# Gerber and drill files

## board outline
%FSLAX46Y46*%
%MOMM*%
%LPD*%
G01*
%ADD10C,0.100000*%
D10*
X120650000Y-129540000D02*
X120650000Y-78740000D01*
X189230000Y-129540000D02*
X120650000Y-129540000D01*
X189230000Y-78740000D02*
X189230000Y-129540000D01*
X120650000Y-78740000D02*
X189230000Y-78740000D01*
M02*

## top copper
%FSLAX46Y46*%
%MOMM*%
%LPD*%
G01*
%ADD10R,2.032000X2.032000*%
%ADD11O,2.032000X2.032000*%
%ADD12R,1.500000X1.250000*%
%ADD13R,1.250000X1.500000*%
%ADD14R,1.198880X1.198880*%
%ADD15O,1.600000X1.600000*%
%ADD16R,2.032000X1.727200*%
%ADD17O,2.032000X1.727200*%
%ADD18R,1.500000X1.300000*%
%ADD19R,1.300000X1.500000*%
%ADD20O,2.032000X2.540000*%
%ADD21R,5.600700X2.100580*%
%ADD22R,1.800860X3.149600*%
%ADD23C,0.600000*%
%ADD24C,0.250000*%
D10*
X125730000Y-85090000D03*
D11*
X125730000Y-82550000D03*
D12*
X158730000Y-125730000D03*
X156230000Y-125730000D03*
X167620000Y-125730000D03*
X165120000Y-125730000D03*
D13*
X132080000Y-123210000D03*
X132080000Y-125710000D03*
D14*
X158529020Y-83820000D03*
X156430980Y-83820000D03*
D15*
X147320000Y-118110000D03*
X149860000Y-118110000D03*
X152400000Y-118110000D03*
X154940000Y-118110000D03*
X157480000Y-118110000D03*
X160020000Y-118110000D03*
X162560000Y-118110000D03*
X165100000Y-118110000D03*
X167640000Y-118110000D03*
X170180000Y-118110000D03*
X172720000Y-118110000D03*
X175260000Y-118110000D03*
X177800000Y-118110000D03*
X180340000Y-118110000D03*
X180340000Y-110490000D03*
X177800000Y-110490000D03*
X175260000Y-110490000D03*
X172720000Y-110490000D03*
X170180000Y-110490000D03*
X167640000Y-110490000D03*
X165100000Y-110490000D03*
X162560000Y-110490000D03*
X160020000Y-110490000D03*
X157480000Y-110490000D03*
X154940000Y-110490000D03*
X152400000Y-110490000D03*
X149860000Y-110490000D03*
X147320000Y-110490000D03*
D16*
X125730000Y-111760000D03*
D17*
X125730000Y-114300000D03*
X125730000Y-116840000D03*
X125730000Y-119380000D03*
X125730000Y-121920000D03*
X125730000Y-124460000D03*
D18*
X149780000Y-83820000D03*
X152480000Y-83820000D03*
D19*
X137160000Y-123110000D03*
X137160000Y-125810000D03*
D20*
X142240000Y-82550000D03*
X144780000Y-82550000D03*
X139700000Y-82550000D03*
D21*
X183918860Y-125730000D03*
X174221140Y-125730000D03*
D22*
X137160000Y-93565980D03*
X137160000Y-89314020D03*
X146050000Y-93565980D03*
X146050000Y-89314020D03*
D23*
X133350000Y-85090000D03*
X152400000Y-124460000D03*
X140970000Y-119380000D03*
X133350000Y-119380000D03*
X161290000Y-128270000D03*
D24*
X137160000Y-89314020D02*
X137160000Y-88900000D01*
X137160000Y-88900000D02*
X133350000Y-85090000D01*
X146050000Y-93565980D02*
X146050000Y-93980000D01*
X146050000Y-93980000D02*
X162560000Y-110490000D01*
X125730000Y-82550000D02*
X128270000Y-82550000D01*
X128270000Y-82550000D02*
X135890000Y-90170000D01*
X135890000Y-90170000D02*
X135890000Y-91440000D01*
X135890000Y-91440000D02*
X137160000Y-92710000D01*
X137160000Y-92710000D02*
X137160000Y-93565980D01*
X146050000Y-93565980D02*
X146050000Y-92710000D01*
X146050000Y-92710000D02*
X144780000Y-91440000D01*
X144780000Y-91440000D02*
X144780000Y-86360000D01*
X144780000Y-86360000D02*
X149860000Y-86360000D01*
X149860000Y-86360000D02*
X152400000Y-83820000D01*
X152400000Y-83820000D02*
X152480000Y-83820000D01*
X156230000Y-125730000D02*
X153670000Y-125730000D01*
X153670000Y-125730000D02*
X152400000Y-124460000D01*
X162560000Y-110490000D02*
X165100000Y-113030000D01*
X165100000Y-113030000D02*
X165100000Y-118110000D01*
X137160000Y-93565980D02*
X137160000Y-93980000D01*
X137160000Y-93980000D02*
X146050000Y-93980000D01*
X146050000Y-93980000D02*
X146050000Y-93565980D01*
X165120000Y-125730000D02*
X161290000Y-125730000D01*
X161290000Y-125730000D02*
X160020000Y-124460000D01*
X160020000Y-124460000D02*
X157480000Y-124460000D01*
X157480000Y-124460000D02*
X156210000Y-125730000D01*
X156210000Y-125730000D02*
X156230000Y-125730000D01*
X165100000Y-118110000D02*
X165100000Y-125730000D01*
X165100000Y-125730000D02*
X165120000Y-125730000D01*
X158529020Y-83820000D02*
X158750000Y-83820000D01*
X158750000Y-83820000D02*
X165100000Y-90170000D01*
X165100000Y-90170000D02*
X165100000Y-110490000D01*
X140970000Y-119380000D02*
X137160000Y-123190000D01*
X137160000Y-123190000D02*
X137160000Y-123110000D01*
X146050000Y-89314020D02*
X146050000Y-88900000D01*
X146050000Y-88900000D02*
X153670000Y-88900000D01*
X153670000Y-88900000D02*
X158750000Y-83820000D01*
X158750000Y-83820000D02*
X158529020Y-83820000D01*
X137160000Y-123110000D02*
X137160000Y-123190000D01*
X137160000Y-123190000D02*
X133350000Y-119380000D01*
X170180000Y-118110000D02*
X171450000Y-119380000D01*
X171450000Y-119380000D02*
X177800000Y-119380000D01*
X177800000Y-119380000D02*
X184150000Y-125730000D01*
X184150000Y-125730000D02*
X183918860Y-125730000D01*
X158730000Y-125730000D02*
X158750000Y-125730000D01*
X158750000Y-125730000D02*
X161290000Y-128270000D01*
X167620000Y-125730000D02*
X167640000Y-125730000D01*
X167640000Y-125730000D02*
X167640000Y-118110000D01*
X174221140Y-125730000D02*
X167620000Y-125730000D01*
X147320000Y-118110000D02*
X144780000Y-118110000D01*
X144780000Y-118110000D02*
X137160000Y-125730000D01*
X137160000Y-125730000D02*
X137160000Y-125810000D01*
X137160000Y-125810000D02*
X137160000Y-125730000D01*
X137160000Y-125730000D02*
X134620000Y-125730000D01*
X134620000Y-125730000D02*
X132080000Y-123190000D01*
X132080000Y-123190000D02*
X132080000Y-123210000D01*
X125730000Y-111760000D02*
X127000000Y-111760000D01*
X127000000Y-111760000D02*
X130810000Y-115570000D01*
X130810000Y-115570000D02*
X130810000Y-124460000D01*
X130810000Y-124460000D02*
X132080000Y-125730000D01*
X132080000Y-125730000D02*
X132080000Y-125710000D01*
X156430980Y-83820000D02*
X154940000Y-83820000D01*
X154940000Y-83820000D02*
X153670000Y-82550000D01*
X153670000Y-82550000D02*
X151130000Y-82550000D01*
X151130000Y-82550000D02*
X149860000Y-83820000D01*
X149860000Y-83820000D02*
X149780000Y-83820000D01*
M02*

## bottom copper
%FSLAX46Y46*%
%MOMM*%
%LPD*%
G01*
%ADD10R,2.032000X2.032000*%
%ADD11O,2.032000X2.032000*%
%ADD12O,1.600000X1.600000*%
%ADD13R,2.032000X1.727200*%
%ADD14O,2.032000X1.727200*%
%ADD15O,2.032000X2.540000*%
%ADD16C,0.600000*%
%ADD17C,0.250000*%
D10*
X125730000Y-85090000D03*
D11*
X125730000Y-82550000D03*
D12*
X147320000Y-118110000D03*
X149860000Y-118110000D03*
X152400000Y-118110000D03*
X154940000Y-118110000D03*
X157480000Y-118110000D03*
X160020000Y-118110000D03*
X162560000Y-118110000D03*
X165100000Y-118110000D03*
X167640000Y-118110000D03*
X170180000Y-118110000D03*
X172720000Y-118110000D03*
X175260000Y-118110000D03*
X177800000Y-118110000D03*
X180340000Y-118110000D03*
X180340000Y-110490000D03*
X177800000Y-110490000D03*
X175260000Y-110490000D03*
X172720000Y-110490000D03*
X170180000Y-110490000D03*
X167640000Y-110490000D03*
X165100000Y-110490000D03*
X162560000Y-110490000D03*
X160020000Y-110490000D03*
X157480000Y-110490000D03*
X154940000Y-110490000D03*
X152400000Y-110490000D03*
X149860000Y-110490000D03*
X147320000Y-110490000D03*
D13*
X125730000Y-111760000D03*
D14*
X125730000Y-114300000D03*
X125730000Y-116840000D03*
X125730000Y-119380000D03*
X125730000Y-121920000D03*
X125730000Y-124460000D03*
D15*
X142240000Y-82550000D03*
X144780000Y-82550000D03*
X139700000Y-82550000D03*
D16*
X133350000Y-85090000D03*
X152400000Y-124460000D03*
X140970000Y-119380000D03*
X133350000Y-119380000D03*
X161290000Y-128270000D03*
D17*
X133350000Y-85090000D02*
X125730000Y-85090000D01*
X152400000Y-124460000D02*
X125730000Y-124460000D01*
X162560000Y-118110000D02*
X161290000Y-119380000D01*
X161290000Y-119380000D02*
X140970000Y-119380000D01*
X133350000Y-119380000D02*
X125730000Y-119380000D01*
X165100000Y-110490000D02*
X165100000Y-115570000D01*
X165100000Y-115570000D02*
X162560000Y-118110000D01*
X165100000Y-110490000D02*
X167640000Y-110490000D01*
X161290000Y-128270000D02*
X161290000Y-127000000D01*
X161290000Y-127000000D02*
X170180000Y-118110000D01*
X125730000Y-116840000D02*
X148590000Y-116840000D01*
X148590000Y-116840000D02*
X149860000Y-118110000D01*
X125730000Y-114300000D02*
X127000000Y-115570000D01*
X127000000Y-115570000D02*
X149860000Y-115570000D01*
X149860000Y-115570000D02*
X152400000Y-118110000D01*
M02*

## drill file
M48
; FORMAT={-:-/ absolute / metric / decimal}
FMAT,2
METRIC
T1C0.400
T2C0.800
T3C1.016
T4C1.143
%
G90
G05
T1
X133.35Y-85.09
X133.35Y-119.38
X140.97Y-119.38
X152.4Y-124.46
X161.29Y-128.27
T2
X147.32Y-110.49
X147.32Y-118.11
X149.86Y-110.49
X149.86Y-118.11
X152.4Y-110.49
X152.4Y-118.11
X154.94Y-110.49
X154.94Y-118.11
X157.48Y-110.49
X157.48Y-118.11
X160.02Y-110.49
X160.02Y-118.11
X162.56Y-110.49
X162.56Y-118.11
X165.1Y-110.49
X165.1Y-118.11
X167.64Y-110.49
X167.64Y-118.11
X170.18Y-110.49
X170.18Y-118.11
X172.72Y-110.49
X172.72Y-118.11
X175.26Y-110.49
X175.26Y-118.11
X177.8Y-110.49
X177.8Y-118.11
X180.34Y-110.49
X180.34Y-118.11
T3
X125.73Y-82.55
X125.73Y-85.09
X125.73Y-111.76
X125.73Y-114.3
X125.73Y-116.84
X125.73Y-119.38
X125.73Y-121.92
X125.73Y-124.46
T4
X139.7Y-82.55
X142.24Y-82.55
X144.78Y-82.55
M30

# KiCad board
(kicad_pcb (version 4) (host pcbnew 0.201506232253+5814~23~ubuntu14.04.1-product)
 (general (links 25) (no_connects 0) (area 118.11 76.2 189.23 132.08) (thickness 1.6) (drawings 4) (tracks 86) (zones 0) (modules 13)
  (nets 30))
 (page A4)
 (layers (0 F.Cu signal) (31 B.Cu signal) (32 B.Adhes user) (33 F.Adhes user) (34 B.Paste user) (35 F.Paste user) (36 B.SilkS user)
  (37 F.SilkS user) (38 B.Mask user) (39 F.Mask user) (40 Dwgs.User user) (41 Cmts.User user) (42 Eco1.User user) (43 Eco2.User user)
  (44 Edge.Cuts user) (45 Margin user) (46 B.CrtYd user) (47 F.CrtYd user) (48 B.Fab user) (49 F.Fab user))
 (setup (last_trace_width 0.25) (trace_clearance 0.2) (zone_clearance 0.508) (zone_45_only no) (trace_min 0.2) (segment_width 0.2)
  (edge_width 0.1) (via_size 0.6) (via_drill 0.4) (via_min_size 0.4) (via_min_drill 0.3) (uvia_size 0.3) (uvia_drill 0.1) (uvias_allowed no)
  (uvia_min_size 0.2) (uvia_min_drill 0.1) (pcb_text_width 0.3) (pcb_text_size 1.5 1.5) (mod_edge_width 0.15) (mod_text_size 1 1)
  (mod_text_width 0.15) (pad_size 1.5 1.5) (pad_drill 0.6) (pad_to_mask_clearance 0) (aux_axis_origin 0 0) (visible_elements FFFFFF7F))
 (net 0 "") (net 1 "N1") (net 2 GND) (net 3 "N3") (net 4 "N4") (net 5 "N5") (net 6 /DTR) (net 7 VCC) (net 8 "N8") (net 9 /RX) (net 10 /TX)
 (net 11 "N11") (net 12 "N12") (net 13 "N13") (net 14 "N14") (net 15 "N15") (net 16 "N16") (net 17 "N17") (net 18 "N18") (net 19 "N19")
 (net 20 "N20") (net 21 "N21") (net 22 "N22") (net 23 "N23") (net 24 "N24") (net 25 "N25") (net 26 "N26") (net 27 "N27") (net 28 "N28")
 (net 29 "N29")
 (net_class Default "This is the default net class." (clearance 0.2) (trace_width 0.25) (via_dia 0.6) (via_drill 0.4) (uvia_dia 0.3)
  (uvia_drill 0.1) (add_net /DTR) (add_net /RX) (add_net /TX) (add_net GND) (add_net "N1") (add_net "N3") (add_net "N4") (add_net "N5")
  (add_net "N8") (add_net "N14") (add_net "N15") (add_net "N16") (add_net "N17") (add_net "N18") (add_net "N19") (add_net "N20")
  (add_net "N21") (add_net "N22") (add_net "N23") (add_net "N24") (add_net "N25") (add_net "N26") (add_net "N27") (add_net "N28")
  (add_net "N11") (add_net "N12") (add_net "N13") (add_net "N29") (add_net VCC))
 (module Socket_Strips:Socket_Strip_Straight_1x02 (layer F.Cu) (at 125.73 85.09 90)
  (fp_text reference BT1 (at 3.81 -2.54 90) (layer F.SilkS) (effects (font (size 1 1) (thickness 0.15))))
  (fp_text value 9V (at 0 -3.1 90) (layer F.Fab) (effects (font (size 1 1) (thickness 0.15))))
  (pad 1 thru_hole rect (at 0 0 90) (size 2.032 2.032) (drill 1.016) (layers *.Cu *.Mask F.SilkS) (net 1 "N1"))
  (pad 2 thru_hole oval (at 2.54 0 90) (size 2.032 2.032) (drill 1.016) (layers *.Cu *.Mask F.SilkS) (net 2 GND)))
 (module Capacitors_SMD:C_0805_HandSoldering (layer F.Cu) (at 157.48 125.73 180)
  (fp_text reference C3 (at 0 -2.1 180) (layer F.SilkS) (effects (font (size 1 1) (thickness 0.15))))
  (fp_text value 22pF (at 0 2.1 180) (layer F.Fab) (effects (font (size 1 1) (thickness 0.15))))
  (pad 1 smd rect (at -1.25 0 180) (size 1.5 1.25) (layers F.Cu F.Paste F.Mask) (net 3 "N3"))
  (pad 2 smd rect (at 1.25 0 180) (size 1.5 1.25) (layers F.Cu F.Paste F.Mask) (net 2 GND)))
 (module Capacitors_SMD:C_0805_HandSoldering (layer F.Cu) (at 166.37 125.73 180)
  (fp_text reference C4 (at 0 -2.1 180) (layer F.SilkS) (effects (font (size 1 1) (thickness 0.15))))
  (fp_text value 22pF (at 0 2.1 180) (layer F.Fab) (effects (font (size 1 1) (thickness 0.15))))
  (pad 1 smd rect (at -1.25 0 180) (size 1.5 1.25) (layers F.Cu F.Paste F.Mask) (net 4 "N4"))
  (pad 2 smd rect (at 1.25 0 180) (size 1.5 1.25) (layers F.Cu F.Paste F.Mask) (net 2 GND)))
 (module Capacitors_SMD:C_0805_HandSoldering (layer F.Cu) (at 132.08 124.46 270)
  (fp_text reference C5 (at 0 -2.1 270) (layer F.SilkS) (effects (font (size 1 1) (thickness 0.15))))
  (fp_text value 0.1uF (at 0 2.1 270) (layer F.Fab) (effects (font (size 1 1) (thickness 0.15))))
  (pad 1 smd rect (at -1.25 0 270) (size 1.5 1.25) (layers F.Cu F.Paste F.Mask) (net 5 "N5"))
  (pad 2 smd rect (at 1.25 0 270) (size 1.5 1.25) (layers F.Cu F.Paste F.Mask) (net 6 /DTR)))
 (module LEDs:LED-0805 (layer F.Cu) (at 157.48 83.82)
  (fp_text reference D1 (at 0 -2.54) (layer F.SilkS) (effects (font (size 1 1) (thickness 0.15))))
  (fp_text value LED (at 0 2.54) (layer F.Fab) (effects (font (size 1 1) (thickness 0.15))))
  (pad 2 smd rect (at 1.04902 0 180) (size 1.19888 1.19888) (layers F.Cu F.Paste F.Mask) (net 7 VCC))
  (pad 1 smd rect (at -1.04902 0 180) (size 1.19888 1.19888) (layers F.Cu F.Paste F.Mask) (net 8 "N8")))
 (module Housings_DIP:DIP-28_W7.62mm (layer F.Cu) (at 147.32 118.11 90)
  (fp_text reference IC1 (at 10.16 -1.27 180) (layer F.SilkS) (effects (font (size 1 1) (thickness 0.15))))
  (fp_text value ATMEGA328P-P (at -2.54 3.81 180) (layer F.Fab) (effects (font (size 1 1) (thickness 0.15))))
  (pad 1 thru_hole oval (at 0 0 90) (size 1.6 1.6) (drill 0.8) (layers *.Cu *.Mask F.SilkS) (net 5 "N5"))
  (pad 2 thru_hole oval (at 0 2.54 90) (size 1.6 1.6) (drill 0.8) (layers *.Cu *.Mask F.SilkS) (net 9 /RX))
  (pad 3 thru_hole oval (at 0 5.08 90) (size 1.6 1.6) (drill 0.8) (layers *.Cu *.Mask F.SilkS) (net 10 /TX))
  (pad 4 thru_hole oval (at 0 7.62 90) (size 1.6 1.6) (drill 0.8) (layers *.Cu *.Mask F.SilkS) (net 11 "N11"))
  (pad 5 thru_hole oval (at 0 10.16 90) (size 1.6 1.6) (drill 0.8) (layers *.Cu *.Mask F.SilkS) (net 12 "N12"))
  (pad 6 thru_hole oval (at 0 12.7 90) (size 1.6 1.6) (drill 0.8) (layers *.Cu *.Mask F.SilkS) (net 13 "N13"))
  (pad 7 thru_hole oval (at 0 15.24 90) (size 1.6 1.6) (drill 0.8) (layers *.Cu *.Mask F.SilkS) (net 7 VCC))
  (pad 8 thru_hole oval (at 0 17.78 90) (size 1.6 1.6) (drill 0.8) (layers *.Cu *.Mask F.SilkS) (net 2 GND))
  (pad 9 thru_hole oval (at 0 20.32 90) (size 1.6 1.6) (drill 0.8) (layers *.Cu *.Mask F.SilkS) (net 4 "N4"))
  (pad 10 thru_hole oval (at 0 22.86 90) (size 1.6 1.6) (drill 0.8) (layers *.Cu *.Mask F.SilkS) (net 3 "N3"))
  (pad 11 thru_hole oval (at 0 25.4 90) (size 1.6 1.6) (drill 0.8) (layers *.Cu *.Mask F.SilkS) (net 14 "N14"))
  (pad 12 thru_hole oval (at 0 27.94 90) (size 1.6 1.6) (drill 0.8) (layers *.Cu *.Mask F.SilkS) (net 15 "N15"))
  (pad 13 thru_hole oval (at 0 30.48 90) (size 1.6 1.6) (drill 0.8) (layers *.Cu *.Mask F.SilkS) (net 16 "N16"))
  (pad 14 thru_hole oval (at 0 33.02 90) (size 1.6 1.6) (drill 0.8) (layers *.Cu *.Mask F.SilkS) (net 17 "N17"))
  (pad 15 thru_hole oval (at 7.62 33.02 90) (size 1.6 1.6) (drill 0.8) (layers *.Cu *.Mask F.SilkS) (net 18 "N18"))
  (pad 16 thru_hole oval (at 7.62 30.48 90) (size 1.6 1.6) (drill 0.8) (layers *.Cu *.Mask F.SilkS) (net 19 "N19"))
  (pad 17 thru_hole oval (at 7.62 27.94 90) (size 1.6 1.6) (drill 0.8) (layers *.Cu *.Mask F.SilkS) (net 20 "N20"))
  (pad 18 thru_hole oval (at 7.62 25.4 90) (size 1.6 1.6) (drill 0.8) (layers *.Cu *.Mask F.SilkS) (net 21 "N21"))
  (pad 19 thru_hole oval (at 7.62 22.86 90) (size 1.6 1.6) (drill 0.8) (layers *.Cu *.Mask F.SilkS) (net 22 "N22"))
  (pad 20 thru_hole oval (at 7.62 20.32 90) (size 1.6 1.6) (drill 0.8) (layers *.Cu *.Mask F.SilkS) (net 7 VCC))
  (pad 21 thru_hole oval (at 7.62 17.78 90) (size 1.6 1.6) (drill 0.8) (layers *.Cu *.Mask F.SilkS) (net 7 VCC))
  (pad 22 thru_hole oval (at 7.62 15.24 90) (size 1.6 1.6) (drill 0.8) (layers *.Cu *.Mask F.SilkS) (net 2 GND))
  (pad 23 thru_hole oval (at 7.62 12.7 90) (size 1.6 1.6) (drill 0.8) (layers *.Cu *.Mask F.SilkS) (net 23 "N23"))
  (pad 24 thru_hole oval (at 7.62 10.16 90) (size 1.6 1.6) (drill 0.8) (layers *.Cu *.Mask F.SilkS) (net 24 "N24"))
  (pad 25 thru_hole oval (at 7.62 7.62 90) (size 1.6 1.6) (drill 0.8) (layers *.Cu *.Mask F.SilkS) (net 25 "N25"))
  (pad 26 thru_hole oval (at 7.62 5.08 90) (size 1.6 1.6) (drill 0.8) (layers *.Cu *.Mask F.SilkS) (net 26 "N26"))
  (pad 27 thru_hole oval (at 7.62 2.54 90) (size 1.6 1.6) (drill 0.8) (layers *.Cu *.Mask F.SilkS) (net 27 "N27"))
  (pad 28 thru_hole oval (at 7.62 0 90) (size 1.6 1.6) (drill 0.8) (layers *.Cu *.Mask F.SilkS) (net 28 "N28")))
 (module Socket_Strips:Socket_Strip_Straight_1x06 (layer F.Cu) (at 125.73 111.76 270)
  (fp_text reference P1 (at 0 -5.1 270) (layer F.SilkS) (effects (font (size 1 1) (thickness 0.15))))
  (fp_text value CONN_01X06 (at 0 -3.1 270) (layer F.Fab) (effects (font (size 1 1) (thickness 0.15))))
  (pad 1 thru_hole rect (at 0 0 270) (size 1.7272 2.032) (drill 1.016) (layers *.Cu *.Mask F.SilkS) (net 6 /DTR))
  (pad 2 thru_hole oval (at 2.54 0 270) (size 1.7272 2.032) (drill 1.016) (layers *.Cu *.Mask F.SilkS) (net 10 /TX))
  (pad 3 thru_hole oval (at 5.08 0 270) (size 1.7272 2.032) (drill 1.016) (layers *.Cu *.Mask F.SilkS) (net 9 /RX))
  (pad 4 thru_hole oval (at 7.62 0 270) (size 1.7272 2.032) (drill 1.016) (layers *.Cu *.Mask F.SilkS) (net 7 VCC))
  (pad 5 thru_hole oval (at 10.16 0 270) (size 1.7272 2.032) (drill 1.016) (layers *.Cu *.Mask F.SilkS) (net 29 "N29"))
  (pad 6 thru_hole oval (at 12.7 0 270) (size 1.7272 2.032) (drill 1.016) (layers *.Cu *.Mask F.SilkS) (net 2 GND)))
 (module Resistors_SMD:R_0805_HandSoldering (layer F.Cu) (at 151.13 83.82)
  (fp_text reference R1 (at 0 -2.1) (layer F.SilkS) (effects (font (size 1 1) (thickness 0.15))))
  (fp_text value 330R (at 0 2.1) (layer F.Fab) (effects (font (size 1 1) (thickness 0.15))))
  (pad 1 smd rect (at -1.35 0) (size 1.5 1.3) (layers F.Cu F.Paste F.Mask) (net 8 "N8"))
  (pad 2 smd rect (at 1.35 0) (size 1.5 1.3) (layers F.Cu F.Paste F.Mask) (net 2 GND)))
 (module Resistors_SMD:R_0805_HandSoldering (layer F.Cu) (at 137.16 124.46 270)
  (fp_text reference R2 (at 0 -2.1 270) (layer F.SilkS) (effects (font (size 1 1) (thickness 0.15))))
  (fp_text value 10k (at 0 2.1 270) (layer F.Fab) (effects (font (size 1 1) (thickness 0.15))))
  (pad 1 smd rect (at -1.35 0 270) (size 1.5 1.3) (layers F.Cu F.Paste F.Mask) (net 7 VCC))
  (pad 2 smd rect (at 1.35 0 270) (size 1.5 1.3) (layers F.Cu F.Paste F.Mask) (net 5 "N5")))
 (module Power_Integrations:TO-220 (layer F.Cu) (at 142.24 82.55)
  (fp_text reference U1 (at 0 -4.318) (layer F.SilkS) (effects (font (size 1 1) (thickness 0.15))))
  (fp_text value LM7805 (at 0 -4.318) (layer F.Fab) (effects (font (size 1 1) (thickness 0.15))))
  (pad 2 thru_hole oval (at 0 0) (size 2.032 2.54) (drill 1.143) (layers *.Cu *.Mask F.SilkS))
  (pad 3 thru_hole oval (at 2.54 0) (size 2.032 2.54) (drill 1.143) (layers *.Cu *.Mask F.SilkS))
  (pad 1 thru_hole oval (at -2.54 0) (size 2.032 2.54) (drill 1.143) (layers *.Cu *.Mask F.SilkS)))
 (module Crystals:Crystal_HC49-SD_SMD (layer F.Cu) (at 179.07 125.73 180)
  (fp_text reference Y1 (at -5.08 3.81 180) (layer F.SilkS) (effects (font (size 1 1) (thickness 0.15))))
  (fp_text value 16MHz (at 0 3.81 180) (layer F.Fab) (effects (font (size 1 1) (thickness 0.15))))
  (pad 1 smd rect (at -4.84886 0 180) (size 5.6007 2.10058) (layers F.Cu F.Paste F.Mask) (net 3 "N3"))
  (pad 2 smd rect (at 4.84886 0 180) (size 5.6007 2.10058) (layers F.Cu F.Paste F.Mask) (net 4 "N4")))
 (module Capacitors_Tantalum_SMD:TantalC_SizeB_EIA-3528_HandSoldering (layer F.Cu) (at 137.16 91.44 270)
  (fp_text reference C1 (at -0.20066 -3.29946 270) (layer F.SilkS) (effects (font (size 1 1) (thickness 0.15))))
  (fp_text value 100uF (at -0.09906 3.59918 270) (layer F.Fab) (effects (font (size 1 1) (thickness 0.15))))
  (pad 2 smd rect (at 2.12598 0 270) (size 3.1496 1.80086) (layers F.Cu F.Paste F.Mask) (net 2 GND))
  (pad 1 smd rect (at -2.12598 0 270) (size 3.1496 1.80086) (layers F.Cu F.Paste F.Mask) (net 1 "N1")))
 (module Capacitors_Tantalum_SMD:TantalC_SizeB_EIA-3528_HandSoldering (layer F.Cu) (at 146.05 91.44 270)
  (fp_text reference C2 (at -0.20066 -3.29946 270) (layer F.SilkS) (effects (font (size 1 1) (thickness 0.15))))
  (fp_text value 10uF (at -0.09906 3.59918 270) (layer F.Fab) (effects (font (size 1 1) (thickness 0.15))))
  (pad 2 smd rect (at 2.12598 0 270) (size 3.1496 1.80086) (layers F.Cu F.Paste F.Mask) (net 2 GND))
  (pad 1 smd rect (at -2.12598 0 270) (size 3.1496 1.80086) (layers F.Cu F.Paste F.Mask) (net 7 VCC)))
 (gr_line (start 120.65 129.54) (end 120.65 78.74) (angle 90) (layer Edge.Cuts) (width 0.1))
 (gr_line (start 189.23 129.54) (end 120.65 129.54) (angle 90) (layer Edge.Cuts) (width 0.1))
 (gr_line (start 189.23 78.74) (end 189.23 129.54) (angle 90) (layer Edge.Cuts) (width 0.1))
 (gr_line (start 120.65 78.74) (end 189.23 78.74) (angle 90) (layer Edge.Cuts) (width 0.1))
 (segment (start 137.16 89.31402) (end 137.16 88.9) (width 0.25) (layer F.Cu) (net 1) (status 80000))
 (segment (start 137.16 88.9) (end 133.35 85.09) (width 0.25) (layer F.Cu) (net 1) (status 80000))
 (segment (start 133.35 85.09) (end 125.73 85.09) (width 0.25) (layer B.Cu) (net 1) (status 80000))
 (segment (start 146.05 93.56598) (end 146.05 93.98) (width 0.25) (layer F.Cu) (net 2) (status 80000))
 (segment (start 146.05 93.98) (end 162.56 110.49) (width 0.25) (layer F.Cu) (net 2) (status 80000))
 (segment (start 125.73 82.55) (end 128.27 82.55) (width 0.25) (layer F.Cu) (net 2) (status 80000))
 (segment (start 128.27 82.55) (end 135.89 90.17) (width 0.25) (layer F.Cu) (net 2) (status 80000))
 (segment (start 135.89 90.17) (end 135.89 91.44) (width 0.25) (layer F.Cu) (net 2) (status 80000))
 (segment (start 135.89 91.44) (end 137.16 92.71) (width 0.25) (layer F.Cu) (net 2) (status 80000))
 (segment (start 137.16 92.71) (end 137.16 93.56598) (width 0.25) (layer F.Cu) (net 2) (status 80000))
 (segment (start 146.05 93.56598) (end 146.05 92.71) (width 0.25) (layer F.Cu) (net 2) (status 80000))
 (segment (start 146.05 92.71) (end 144.78 91.44) (width 0.25) (layer F.Cu) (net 2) (status 80000))
 (segment (start 144.78 91.44) (end 144.78 86.36) (width 0.25) (layer F.Cu) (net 2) (status 80000))
 (segment (start 144.78 86.36) (end 149.86 86.36) (width 0.25) (layer F.Cu) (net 2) (status 80000))
 (segment (start 149.86 86.36) (end 152.4 83.82) (width 0.25) (layer F.Cu) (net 2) (status 80000))
 (segment (start 152.4 83.82) (end 152.48 83.82) (width 0.25) (layer F.Cu) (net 2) (status 80000))
 (segment (start 156.23 125.73) (end 153.67 125.73) (width 0.25) (layer F.Cu) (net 2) (status 80000))
 (segment (start 153.67 125.73) (end 152.4 124.46) (width 0.25) (layer F.Cu) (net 2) (status 80000))
 (segment (start 152.4 124.46) (end 125.73 124.46) (width 0.25) (layer B.Cu) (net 2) (status 80000))
 (segment (start 162.56 110.49) (end 165.1 113.03) (width 0.25) (layer F.Cu) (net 2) (status 80000))
 (segment (start 165.1 113.03) (end 165.1 118.11) (width 0.25) (layer F.Cu) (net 2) (status 80000))
 (segment (start 137.16 93.56598) (end 137.16 93.98) (width 0.25) (layer F.Cu) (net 2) (status 80000))
 (segment (start 137.16 93.98) (end 146.05 93.98) (width 0.25) (layer F.Cu) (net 2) (status 80000))
 (segment (start 146.05 93.98) (end 146.05 93.56598) (width 0.25) (layer F.Cu) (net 2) (status 80000))
 (segment (start 165.12 125.73) (end 161.29 125.73) (width 0.25) (layer F.Cu) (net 2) (status 80000))
 (segment (start 161.29 125.73) (end 160.02 124.46) (width 0.25) (layer F.Cu) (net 2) (status 80000))
 (segment (start 160.02 124.46) (end 157.48 124.46) (width 0.25) (layer F.Cu) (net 2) (status 80000))
 (segment (start 157.48 124.46) (end 156.21 125.73) (width 0.25) (layer F.Cu) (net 2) (status 80000))
 (segment (start 156.21 125.73) (end 156.23 125.73) (width 0.25) (layer F.Cu) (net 2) (status 80000))
 (segment (start 165.1 118.11) (end 165.1 125.73) (width 0.25) (layer F.Cu) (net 2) (status 80000))
 (segment (start 165.1 125.73) (end 165.12 125.73) (width 0.25) (layer F.Cu) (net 2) (status 80000))
 (segment (start 158.52902 83.82) (end 158.75 83.82) (width 0.25) (layer F.Cu) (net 7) (status 80000))
 (segment (start 158.75 83.82) (end 165.1 90.17) (width 0.25) (layer F.Cu) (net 7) (status 80000))
 (segment (start 165.1 90.17) (end 165.1 110.49) (width 0.25) (layer F.Cu) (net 7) (status 80000))
 (segment (start 162.56 118.11) (end 161.29 119.38) (width 0.25) (layer B.Cu) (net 7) (status 80000))
 (segment (start 161.29 119.38) (end 140.97 119.38) (width 0.25) (layer B.Cu) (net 7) (status 80000))
 (segment (start 140.97 119.38) (end 137.16 123.19) (width 0.25) (layer F.Cu) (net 7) (status 80000))
 (segment (start 137.16 123.19) (end 137.16 123.11) (width 0.25) (layer F.Cu) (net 7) (status 80000))
 (segment (start 146.05 89.31402) (end 146.05 88.9) (width 0.25) (layer F.Cu) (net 7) (status 80000))
 (segment (start 146.05 88.9) (end 153.67 88.9) (width 0.25) (layer F.Cu) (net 7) (status 80000))
 (segment (start 153.67 88.9) (end 158.75 83.82) (width 0.25) (layer F.Cu) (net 7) (status 80000))
 (segment (start 158.75 83.82) (end 158.52902 83.82) (width 0.25) (layer F.Cu) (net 7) (status 80000))
 (segment (start 137.16 123.11) (end 137.16 123.19) (width 0.25) (layer F.Cu) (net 7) (status 80000))
 (segment (start 137.16 123.19) (end 133.35 119.38) (width 0.25) (layer F.Cu) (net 7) (status 80000))
 (segment (start 133.35 119.38) (end 125.73 119.38) (width 0.25) (layer B.Cu) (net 7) (status 80000))
 (segment (start 165.1 110.49) (end 165.1 115.57) (width 0.25) (layer B.Cu) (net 7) (status 80000))
 (segment (start 165.1 115.57) (end 162.56 118.11) (width 0.25) (layer B.Cu) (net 7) (status 80000))
 (segment (start 165.1 110.49) (end 167.64 110.49) (width 0.25) (layer B.Cu) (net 7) (status 80000))
 (segment (start 170.18 118.11) (end 171.45 119.38) (width 0.25) (layer F.Cu) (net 3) (status 80000))
 (segment (start 171.45 119.38) (end 177.8 119.38) (width 0.25) (layer F.Cu) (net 3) (status 80000))
 (segment (start 177.8 119.38) (end 184.15 125.73) (width 0.25) (layer F.Cu) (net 3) (status 80000))
 (segment (start 184.15 125.73) (end 183.91886 125.73) (width 0.25) (layer F.Cu) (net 3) (status 80000))
 (segment (start 158.73 125.73) (end 158.75 125.73) (width 0.25) (layer F.Cu) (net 3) (status 80000))
 (segment (start 158.75 125.73) (end 161.29 128.27) (width 0.25) (layer F.Cu) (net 3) (status 80000))
 (segment (start 161.29 128.27) (end 161.29 127) (width 0.25) (layer B.Cu) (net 3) (status 80000))
 (segment (start 161.29 127) (end 170.18 118.11) (width 0.25) (layer B.Cu) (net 3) (status 80000))
 (segment (start 167.62 125.73) (end 167.64 125.73) (width 0.25) (layer F.Cu) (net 4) (status 80000))
 (segment (start 167.64 125.73) (end 167.64 118.11) (width 0.25) (layer F.Cu) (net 4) (status 80000))
 (segment (start 174.22114 125.73) (end 167.62 125.73) (width 0.25) (layer F.Cu) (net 4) (status 80000))
 (segment (start 147.32 118.11) (end 144.78 118.11) (width 0.25) (layer F.Cu) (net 5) (status 80000))
 (segment (start 144.78 118.11) (end 137.16 125.73) (width 0.25) (layer F.Cu) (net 5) (status 80000))
 (segment (start 137.16 125.73) (end 137.16 125.81) (width 0.25) (layer F.Cu) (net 5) (status 80000))
 (segment (start 137.16 125.81) (end 137.16 125.73) (width 0.25) (layer F.Cu) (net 5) (status 80000))
 (segment (start 137.16 125.73) (end 134.62 125.73) (width 0.25) (layer F.Cu) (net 5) (status 80000))
 (segment (start 134.62 125.73) (end 132.08 123.19) (width 0.25) (layer F.Cu) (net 5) (status 80000))
 (segment (start 132.08 123.19) (end 132.08 123.21) (width 0.25) (layer F.Cu) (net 5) (status 80000))
 (segment (start 125.73 111.76) (end 127 111.76) (width 0.25) (layer F.Cu) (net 6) (status 80000))
 (segment (start 127 111.76) (end 130.81 115.57) (width 0.25) (layer F.Cu) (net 6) (status 80000))
 (segment (start 130.81 115.57) (end 130.81 124.46) (width 0.25) (layer F.Cu) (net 6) (status 80000))
 (segment (start 130.81 124.46) (end 132.08 125.73) (width 0.25) (layer F.Cu) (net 6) (status 80000))
 (segment (start 132.08 125.73) (end 132.08 125.71) (width 0.25) (layer F.Cu) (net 6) (status 80000))
 (segment (start 156.43098 83.82) (end 154.94 83.82) (width 0.25) (layer F.Cu) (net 8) (status 80000))
 (segment (start 154.94 83.82) (end 153.67 82.55) (width 0.25) (layer F.Cu) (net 8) (status 80000))
 (segment (start 153.67 82.55) (end 151.13 82.55) (width 0.25) (layer F.Cu) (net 8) (status 80000))
 (segment (start 151.13 82.55) (end 149.86 83.82) (width 0.25) (layer F.Cu) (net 8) (status 80000))
 (segment (start 149.86 83.82) (end 149.78 83.82) (width 0.25) (layer F.Cu) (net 8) (status 80000))
 (segment (start 125.73 116.84) (end 148.59 116.84) (width 0.25) (layer B.Cu) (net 9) (status 80000))
 (segment (start 148.59 116.84) (end 149.86 118.11) (width 0.25) (layer B.Cu) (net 9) (status 80000))
 (segment (start 125.73 114.3) (end 127 115.57) (width 0.25) (layer B.Cu) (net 10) (status 80000))
 (segment (start 127 115.57) (end 149.86 115.57) (width 0.25) (layer B.Cu) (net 10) (status 80000))
 (segment (start 149.86 115.57) (end 152.4 118.11) (width 0.25) (layer B.Cu) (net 10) (status 80000))
 (via (at 133.35 85.09) (size 0.6) (layers F.Cu B.Cu) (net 1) (status 80000))
 (via (at 152.4 124.46) (size 0.6) (layers F.Cu B.Cu) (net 2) (status 80000))
 (via (at 140.97 119.38) (size 0.6) (layers F.Cu B.Cu) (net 7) (status 80000))
 (via (at 133.35 119.38) (size 0.6) (layers F.Cu B.Cu) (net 7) (status 80000))
 (via (at 161.29 128.27) (size 0.6) (layers F.Cu B.Cu) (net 3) (status 80000)))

